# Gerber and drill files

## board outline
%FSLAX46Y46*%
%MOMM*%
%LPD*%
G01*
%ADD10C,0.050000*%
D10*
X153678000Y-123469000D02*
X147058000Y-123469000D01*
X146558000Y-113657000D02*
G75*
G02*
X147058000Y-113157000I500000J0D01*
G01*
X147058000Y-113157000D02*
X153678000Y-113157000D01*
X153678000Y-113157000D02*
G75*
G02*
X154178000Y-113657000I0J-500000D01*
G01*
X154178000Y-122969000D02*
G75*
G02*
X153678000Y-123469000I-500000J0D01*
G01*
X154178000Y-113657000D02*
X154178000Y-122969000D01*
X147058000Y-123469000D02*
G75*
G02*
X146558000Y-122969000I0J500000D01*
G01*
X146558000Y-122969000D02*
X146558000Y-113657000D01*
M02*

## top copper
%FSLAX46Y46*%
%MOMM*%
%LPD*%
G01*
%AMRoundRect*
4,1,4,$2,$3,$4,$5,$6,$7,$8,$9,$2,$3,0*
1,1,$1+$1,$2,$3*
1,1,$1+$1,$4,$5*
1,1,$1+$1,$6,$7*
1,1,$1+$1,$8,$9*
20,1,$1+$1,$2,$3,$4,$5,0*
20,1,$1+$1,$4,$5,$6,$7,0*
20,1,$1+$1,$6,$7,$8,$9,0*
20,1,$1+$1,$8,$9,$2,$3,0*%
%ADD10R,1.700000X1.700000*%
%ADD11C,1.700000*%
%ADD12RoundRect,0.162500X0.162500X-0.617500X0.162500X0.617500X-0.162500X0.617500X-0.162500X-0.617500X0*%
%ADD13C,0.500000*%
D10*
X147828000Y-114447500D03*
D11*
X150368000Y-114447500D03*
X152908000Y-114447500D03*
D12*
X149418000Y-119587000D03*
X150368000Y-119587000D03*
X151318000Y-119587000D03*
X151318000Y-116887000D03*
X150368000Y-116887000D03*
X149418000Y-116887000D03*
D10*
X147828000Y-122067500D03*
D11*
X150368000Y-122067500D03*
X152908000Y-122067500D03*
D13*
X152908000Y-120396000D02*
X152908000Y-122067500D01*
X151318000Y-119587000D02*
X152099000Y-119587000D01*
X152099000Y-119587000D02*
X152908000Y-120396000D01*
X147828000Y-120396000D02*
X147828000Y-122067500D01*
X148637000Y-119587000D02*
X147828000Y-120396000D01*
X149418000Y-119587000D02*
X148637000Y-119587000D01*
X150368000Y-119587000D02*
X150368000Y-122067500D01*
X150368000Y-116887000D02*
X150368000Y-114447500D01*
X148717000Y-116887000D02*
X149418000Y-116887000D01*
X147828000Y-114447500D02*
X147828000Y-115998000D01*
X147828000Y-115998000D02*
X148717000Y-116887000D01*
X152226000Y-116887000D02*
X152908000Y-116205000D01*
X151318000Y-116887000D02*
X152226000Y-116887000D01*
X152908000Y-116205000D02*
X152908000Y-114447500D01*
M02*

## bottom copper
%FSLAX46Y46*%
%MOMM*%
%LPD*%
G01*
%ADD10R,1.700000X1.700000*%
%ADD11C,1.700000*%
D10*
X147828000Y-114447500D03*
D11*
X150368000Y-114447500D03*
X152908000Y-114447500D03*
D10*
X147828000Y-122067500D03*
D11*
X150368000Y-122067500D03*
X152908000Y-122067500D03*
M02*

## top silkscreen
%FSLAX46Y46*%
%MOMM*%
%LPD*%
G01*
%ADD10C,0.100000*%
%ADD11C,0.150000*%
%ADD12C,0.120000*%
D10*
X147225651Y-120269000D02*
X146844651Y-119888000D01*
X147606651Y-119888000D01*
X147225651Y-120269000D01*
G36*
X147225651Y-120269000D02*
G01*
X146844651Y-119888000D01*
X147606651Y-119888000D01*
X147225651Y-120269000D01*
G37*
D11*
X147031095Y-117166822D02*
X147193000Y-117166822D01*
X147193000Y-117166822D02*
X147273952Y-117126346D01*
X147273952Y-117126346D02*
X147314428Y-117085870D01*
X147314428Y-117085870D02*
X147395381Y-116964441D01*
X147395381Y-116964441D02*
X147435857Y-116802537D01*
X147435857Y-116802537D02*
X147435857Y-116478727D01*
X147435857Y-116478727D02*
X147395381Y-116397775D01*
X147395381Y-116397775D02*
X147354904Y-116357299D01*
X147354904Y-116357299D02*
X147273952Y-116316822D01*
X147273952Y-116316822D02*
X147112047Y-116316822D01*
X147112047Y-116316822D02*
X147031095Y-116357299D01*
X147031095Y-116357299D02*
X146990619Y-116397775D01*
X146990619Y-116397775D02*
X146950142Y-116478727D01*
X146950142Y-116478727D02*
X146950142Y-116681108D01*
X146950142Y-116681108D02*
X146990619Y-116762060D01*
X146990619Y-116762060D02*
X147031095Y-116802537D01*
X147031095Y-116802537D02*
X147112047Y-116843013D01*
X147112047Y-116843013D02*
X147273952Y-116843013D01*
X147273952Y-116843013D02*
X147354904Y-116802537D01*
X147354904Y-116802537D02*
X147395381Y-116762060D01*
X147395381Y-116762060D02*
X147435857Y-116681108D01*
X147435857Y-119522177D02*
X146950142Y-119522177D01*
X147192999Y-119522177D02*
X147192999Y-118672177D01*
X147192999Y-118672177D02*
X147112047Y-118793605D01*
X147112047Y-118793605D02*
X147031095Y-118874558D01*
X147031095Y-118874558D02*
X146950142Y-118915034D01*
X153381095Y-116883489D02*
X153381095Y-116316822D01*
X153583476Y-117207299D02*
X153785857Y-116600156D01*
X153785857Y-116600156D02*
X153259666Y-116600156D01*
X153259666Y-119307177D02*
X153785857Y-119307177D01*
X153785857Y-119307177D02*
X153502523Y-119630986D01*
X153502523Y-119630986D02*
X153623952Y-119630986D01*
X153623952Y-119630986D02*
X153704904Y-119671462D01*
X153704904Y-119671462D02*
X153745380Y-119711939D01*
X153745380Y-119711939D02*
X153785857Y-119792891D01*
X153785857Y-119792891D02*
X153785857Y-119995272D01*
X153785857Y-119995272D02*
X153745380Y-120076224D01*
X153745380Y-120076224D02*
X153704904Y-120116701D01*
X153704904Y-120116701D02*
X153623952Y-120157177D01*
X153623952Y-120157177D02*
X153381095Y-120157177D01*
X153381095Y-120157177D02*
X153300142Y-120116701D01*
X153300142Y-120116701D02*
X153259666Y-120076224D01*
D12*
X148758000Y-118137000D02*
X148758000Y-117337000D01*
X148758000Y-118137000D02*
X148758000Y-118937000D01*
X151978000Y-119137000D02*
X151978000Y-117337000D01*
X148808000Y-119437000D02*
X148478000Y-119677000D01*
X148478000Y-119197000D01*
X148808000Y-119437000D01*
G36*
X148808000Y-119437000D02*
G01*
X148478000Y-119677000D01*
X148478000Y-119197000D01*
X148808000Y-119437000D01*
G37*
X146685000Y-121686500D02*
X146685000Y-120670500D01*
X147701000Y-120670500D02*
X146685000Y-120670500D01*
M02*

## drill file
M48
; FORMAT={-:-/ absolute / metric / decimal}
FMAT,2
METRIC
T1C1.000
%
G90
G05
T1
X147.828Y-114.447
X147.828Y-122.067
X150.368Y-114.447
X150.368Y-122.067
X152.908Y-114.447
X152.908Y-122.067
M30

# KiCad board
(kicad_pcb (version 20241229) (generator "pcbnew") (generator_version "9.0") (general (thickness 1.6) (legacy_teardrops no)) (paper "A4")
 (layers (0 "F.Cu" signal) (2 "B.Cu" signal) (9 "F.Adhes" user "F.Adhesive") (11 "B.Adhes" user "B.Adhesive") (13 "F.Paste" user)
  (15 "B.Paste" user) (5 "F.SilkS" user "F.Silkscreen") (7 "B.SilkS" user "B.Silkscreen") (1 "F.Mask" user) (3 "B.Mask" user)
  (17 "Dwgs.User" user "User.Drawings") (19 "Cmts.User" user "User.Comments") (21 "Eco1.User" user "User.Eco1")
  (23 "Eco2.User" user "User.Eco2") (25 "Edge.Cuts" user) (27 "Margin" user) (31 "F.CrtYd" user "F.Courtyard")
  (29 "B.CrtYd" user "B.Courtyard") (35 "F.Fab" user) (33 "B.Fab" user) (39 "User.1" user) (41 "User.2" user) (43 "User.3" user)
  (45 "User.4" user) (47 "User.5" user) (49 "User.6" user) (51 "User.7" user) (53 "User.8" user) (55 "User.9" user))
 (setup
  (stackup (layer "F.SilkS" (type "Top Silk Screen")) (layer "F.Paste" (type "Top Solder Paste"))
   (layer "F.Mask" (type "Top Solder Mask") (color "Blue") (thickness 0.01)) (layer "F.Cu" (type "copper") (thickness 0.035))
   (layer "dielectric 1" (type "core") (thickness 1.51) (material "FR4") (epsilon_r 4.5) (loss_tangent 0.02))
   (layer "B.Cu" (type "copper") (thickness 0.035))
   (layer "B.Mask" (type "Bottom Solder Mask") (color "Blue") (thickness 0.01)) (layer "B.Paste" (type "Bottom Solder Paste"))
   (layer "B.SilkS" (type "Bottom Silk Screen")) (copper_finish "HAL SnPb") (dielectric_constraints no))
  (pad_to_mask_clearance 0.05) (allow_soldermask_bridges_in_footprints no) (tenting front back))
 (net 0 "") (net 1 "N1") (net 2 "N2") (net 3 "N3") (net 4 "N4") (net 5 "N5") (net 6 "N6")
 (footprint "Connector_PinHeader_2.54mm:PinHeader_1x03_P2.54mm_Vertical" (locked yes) (layer "F.Cu") (at 147.828 114.4475 90)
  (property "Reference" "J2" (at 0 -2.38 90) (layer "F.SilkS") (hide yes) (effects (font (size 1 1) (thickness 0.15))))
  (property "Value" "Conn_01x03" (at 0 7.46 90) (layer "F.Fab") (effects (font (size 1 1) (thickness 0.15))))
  (pad "1" thru_hole rect (at 0 0 90) (size 1.7 1.7) (drill 1) (layers "*.Cu" "*.Mask") (remove_unused_layers no) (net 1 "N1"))
  (pad "2" thru_hole circle (at 0 2.54 90) (size 1.7 1.7) (drill 1) (layers "*.Cu" "*.Mask") (remove_unused_layers no) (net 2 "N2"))
  (pad "3" thru_hole circle (at 0 5.08 90) (size 1.7 1.7) (drill 1) (layers "*.Cu" "*.Mask") (remove_unused_layers no) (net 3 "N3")))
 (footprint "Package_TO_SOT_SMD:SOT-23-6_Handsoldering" (layer "F.Cu") (at 150.368 118.237 90)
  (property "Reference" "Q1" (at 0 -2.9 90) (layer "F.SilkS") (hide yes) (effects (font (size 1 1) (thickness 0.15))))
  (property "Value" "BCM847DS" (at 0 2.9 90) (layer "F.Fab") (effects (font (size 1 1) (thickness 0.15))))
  (fp_line (start 0.1 -1.61) (end 0.9 -1.61) (stroke (width 0.12) (type solid)) (layer "F.SilkS"))
  (fp_line (start 0.1 -1.61) (end -0.7 -1.61) (stroke (width 0.12) (type solid)) (layer "F.SilkS"))
  (fp_line (start -0.9 1.61) (end 0.9 1.61) (stroke (width 0.12) (type solid)) (layer "F.SilkS"))
  (fp_poly
   (pts (xy -1.2 -1.56) (xy -1.44 -1.89) (xy -0.96 -1.89) (xy -1.2 -1.56)) (stroke (width 0.12) (type solid)) (fill yes) (layer "F.SilkS"))
  (pad "1" smd roundrect (at -1.35 -0.95 90) (size 1.56 0.65) (layers "F.Cu" "F.Mask" "F.Paste") (roundrect_rratio 0.25) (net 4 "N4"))
  (pad "2" smd roundrect (at -1.35 0 90) (size 1.56 0.65) (layers "F.Cu" "F.Mask" "F.Paste") (roundrect_rratio 0.25) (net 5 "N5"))
  (pad "3" smd roundrect (at -1.35 0.95 90) (size 1.56 0.65) (layers "F.Cu" "F.Mask" "F.Paste") (roundrect_rratio 0.25) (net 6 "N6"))
  (pad "4" smd roundrect (at 1.35 0.95 90) (size 1.56 0.65) (layers "F.Cu" "F.Mask" "F.Paste") (roundrect_rratio 0.25) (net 3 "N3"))
  (pad "5" smd roundrect (at 1.35 0 90) (size 1.56 0.65) (layers "F.Cu" "F.Mask" "F.Paste") (roundrect_rratio 0.25) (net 2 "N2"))
  (pad "6" smd roundrect (at 1.35 -0.95 90) (size 1.56 0.65) (layers "F.Cu" "F.Mask" "F.Paste") (roundrect_rratio 0.25) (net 1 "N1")))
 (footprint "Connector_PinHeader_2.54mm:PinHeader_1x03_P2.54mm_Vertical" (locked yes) (layer "F.Cu") (at 147.828 122.0675 90)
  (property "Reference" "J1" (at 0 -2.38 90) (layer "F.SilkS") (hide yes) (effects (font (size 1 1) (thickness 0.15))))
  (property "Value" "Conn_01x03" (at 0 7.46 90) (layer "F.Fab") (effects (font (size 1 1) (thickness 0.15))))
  (fp_line (start 0.381 -1.143) (end 1.397 -1.143) (stroke (width 0.12) (type solid)) (layer "F.SilkS"))
  (fp_line (start 1.397 -0.127) (end 1.397 -1.143) (stroke (width 0.12) (type solid)) (layer "F.SilkS"))
  (pad "1" thru_hole rect (at 0 0 90) (size 1.7 1.7) (drill 1) (layers "*.Cu" "*.Mask") (remove_unused_layers no) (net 4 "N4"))
  (pad "2" thru_hole circle (at 0 2.54 90) (size 1.7 1.7) (drill 1) (layers "*.Cu" "*.Mask") (remove_unused_layers no) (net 5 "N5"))
  (pad "3" thru_hole circle (at 0 5.08 90) (size 1.7 1.7) (drill 1) (layers "*.Cu" "*.Mask") (remove_unused_layers no) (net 6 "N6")))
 (gr_poly
  (pts (xy 147.225651 120.269) (xy 146.844651 119.888) (xy 147.606651 119.888)) (stroke (width 0.1) (type solid)) (fill yes)
  (layer "F.SilkS"))
 (gr_line (start 153.678 123.469) (end 147.058 123.469) (stroke (width 0.05) (type default)) (locked yes) (layer "Edge.Cuts"))
 (gr_arc (start 146.558 113.657) (mid 146.704447 113.303447) (end 147.058 113.157) (stroke (width 0.05) (type default)) (locked yes)
  (layer "Edge.Cuts"))
 (gr_line (start 147.058 113.157) (end 153.678 113.157) (stroke (width 0.05) (type default)) (locked yes) (layer "Edge.Cuts"))
 (gr_arc (start 153.678 113.157) (mid 154.031553 113.303447) (end 154.178 113.657) (stroke (width 0.05) (type default)) (locked yes)
  (layer "Edge.Cuts"))
 (gr_arc (start 154.178 122.969) (mid 154.031553 123.322553) (end 153.678 123.469) (stroke (width 0.05) (type default)) (locked yes)
  (layer "Edge.Cuts"))
 (gr_line (start 154.178 113.657) (end 154.178 122.969) (stroke (width 0.05) (type default)) (locked yes) (layer "Edge.Cuts"))
 (gr_arc (start 147.058 123.469) (mid 146.704447 123.322553) (end 146.558 122.969) (stroke (width 0.05) (type default)) (locked yes)
  (layer "Edge.Cuts"))
 (gr_line (start 146.558 122.969) (end 146.558 113.657) (stroke (width 0.05) (type default)) (locked yes) (layer "Edge.Cuts"))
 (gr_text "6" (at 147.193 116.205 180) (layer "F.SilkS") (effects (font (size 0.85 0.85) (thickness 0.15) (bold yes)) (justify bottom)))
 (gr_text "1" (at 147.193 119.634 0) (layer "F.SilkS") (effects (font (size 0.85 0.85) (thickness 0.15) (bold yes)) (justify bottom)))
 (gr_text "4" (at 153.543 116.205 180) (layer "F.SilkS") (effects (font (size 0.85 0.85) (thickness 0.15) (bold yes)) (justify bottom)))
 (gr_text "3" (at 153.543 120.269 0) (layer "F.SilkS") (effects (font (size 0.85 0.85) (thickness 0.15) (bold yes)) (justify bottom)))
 (segment (start 152.908 120.396) (end 152.908 122.0675) (width 0.5) (layer "F.Cu") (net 6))
 (segment (start 151.318 119.587) (end 152.099 119.587) (width 0.5) (layer "F.Cu") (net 6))
 (segment (start 152.099 119.587) (end 152.908 120.396) (width 0.5) (layer "F.Cu") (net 6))
 (segment (start 147.828 120.396) (end 147.828 122.0675) (width 0.5) (layer "F.Cu") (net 4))
 (segment (start 148.637 119.587) (end 147.828 120.396) (width 0.5) (layer "F.Cu") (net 4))
 (segment (start 149.418 119.587) (end 148.637 119.587) (width 0.5) (layer "F.Cu") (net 4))
 (segment (start 150.368 119.587) (end 150.368 122.0675) (width 0.5) (layer "F.Cu") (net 5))
 (segment (start 150.368 116.887) (end 150.368 114.4475) (width 0.5) (layer "F.Cu") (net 2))
 (segment (start 148.717 116.887) (end 149.418 116.887) (width 0.5) (layer "F.Cu") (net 1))
 (segment (start 147.828 114.4475) (end 147.828 115.998) (width 0.5) (layer "F.Cu") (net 1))
 (segment (start 147.828 115.998) (end 148.717 116.887) (width 0.5) (layer "F.Cu") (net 1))
 (segment (start 152.226 116.887) (end 152.908 116.205) (width 0.5) (layer "F.Cu") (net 3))
 (segment (start 151.318 116.887) (end 152.226 116.887) (width 0.5) (layer "F.Cu") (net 3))
 (segment (start 152.908 116.205) (end 152.908 114.4475) (width 0.5) (layer "F.Cu") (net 3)))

